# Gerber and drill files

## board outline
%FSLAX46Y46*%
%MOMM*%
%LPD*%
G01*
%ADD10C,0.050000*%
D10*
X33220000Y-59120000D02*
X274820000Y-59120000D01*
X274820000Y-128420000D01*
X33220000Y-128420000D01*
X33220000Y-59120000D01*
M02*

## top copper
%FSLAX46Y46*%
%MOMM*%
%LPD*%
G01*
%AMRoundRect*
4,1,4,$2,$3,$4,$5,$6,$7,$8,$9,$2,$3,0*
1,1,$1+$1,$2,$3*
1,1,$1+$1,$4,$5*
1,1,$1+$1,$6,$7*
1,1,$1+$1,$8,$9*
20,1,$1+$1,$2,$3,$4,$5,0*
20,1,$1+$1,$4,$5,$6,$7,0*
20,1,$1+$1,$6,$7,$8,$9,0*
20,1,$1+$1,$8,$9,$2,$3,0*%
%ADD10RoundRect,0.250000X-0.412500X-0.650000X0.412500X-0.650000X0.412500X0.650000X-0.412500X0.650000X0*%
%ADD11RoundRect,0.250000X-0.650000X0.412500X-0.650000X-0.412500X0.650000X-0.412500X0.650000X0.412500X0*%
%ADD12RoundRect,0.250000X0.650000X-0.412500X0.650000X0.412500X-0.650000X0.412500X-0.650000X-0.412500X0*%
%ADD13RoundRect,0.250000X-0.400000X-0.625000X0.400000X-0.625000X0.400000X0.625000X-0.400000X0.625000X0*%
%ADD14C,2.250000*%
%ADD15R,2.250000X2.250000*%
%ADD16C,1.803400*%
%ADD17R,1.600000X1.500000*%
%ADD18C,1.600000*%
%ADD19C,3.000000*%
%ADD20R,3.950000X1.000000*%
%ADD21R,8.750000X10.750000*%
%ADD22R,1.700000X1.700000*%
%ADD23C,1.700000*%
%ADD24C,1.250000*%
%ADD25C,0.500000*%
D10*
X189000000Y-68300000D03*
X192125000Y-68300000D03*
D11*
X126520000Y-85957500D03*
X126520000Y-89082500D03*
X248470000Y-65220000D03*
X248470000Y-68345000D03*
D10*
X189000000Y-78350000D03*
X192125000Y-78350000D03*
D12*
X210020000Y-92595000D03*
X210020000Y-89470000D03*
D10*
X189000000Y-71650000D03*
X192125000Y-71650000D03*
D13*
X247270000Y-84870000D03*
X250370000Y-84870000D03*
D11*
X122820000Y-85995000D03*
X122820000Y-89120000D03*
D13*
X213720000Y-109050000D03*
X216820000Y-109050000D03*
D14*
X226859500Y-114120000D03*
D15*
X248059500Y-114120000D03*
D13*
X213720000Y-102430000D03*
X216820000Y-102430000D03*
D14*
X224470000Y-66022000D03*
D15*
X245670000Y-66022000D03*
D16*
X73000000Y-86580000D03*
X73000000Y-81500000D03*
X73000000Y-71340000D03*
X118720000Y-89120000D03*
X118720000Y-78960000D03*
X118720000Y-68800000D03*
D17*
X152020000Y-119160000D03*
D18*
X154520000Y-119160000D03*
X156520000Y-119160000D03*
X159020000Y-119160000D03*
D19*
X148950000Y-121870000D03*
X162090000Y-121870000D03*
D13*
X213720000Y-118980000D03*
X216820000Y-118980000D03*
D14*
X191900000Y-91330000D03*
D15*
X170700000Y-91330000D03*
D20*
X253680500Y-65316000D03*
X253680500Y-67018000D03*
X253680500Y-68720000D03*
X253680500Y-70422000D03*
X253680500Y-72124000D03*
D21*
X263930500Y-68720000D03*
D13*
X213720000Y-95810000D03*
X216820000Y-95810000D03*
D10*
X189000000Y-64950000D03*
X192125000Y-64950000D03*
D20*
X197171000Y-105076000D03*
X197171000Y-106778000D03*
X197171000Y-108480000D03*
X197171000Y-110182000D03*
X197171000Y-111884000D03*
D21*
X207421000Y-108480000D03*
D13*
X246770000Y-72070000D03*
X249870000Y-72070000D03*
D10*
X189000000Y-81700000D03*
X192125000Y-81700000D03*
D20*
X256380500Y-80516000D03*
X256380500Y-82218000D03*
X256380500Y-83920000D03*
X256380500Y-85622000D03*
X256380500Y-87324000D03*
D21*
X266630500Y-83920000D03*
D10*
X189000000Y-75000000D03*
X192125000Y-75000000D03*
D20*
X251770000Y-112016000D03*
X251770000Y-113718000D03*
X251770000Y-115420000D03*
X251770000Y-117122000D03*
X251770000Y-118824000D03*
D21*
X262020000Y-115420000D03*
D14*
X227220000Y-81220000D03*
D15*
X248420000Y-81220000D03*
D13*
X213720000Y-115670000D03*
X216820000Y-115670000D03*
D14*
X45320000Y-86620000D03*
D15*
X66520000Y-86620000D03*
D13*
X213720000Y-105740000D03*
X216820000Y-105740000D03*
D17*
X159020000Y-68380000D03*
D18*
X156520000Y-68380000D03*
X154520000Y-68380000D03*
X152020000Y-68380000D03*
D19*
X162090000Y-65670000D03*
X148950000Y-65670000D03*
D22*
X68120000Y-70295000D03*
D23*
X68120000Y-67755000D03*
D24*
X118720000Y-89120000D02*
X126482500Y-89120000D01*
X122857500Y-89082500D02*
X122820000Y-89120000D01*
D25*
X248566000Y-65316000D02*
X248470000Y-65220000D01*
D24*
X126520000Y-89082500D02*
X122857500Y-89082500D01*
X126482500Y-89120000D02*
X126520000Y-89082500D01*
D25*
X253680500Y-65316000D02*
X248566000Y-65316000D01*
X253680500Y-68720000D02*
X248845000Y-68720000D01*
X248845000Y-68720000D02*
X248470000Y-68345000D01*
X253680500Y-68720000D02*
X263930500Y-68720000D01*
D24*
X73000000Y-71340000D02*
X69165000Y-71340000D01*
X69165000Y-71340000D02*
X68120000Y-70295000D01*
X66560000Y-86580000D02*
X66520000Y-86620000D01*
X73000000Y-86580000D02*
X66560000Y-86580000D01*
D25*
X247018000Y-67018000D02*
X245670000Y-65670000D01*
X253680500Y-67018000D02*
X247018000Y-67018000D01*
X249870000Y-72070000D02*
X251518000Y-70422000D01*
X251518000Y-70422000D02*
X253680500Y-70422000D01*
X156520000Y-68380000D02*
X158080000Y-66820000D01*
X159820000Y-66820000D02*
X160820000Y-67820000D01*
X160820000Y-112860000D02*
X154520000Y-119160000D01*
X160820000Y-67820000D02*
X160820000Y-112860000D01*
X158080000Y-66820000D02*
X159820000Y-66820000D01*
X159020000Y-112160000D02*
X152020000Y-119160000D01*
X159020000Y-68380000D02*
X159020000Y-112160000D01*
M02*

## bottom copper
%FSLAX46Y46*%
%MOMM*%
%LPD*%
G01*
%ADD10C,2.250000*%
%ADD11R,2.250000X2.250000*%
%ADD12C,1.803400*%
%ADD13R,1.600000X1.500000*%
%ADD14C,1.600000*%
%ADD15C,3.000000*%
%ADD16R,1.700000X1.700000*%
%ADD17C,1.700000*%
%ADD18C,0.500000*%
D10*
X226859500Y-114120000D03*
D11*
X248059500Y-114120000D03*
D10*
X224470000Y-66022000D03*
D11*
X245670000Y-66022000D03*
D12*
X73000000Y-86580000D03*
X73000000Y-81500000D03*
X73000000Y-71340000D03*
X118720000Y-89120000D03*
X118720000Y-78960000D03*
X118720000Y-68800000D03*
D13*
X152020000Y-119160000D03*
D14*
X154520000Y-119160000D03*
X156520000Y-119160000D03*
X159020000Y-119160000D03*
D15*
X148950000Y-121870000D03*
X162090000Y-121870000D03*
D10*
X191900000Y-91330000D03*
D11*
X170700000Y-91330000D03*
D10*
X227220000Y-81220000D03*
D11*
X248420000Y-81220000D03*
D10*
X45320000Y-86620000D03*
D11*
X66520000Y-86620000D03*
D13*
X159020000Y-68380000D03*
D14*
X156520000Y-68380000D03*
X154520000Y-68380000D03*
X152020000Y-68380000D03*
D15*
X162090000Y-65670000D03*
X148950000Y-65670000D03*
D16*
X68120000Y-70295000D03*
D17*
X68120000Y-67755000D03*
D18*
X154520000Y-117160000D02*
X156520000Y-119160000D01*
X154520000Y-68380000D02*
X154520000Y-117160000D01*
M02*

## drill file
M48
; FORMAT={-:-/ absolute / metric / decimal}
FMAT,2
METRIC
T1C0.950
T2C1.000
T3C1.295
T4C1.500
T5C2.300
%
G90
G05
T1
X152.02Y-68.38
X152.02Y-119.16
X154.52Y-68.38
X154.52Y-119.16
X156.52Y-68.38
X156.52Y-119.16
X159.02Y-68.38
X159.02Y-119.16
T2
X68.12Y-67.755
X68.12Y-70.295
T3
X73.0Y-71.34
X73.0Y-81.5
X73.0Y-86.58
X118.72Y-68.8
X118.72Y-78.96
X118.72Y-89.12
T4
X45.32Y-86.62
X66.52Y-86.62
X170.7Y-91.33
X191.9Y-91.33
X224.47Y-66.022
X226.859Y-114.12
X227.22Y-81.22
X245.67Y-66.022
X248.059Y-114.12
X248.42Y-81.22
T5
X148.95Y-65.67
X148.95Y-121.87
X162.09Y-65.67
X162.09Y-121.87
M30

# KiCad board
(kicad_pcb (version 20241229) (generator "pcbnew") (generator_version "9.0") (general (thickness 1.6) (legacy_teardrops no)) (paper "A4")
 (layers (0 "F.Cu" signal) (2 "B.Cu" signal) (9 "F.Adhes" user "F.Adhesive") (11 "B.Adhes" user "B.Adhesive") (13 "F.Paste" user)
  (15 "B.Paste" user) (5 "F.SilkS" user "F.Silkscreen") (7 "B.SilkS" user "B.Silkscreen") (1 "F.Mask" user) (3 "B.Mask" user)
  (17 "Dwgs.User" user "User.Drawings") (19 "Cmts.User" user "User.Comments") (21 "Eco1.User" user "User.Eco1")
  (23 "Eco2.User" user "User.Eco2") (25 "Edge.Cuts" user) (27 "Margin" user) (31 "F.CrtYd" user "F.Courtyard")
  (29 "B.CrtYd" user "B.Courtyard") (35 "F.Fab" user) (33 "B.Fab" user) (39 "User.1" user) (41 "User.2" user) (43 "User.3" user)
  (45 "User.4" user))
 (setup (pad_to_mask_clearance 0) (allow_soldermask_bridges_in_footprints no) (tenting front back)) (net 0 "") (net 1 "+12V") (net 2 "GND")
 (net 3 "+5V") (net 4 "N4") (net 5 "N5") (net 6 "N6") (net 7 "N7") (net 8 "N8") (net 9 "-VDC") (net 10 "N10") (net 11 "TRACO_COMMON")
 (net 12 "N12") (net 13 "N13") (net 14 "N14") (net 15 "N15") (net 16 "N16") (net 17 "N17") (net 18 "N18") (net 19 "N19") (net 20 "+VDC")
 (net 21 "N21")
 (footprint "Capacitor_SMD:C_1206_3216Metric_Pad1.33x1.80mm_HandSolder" (layer "F.Cu") (at 190.5625 68.3)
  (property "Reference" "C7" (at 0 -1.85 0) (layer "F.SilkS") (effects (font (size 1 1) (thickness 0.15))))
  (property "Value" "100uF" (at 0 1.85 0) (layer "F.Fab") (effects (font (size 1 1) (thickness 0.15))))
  (pad "1" smd roundrect (at -1.5625 0) (size 1.325 1.8) (layers "F.Cu" "F.Mask" "F.Paste") (roundrect_rratio 0.188679) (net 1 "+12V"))
  (pad "2" smd roundrect (at 1.5625 0) (size 1.325 1.8) (layers "F.Cu" "F.Mask" "F.Paste") (roundrect_rratio 0.188679) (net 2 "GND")))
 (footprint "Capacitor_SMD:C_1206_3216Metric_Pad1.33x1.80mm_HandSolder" (layer "F.Cu") (at 126.52 87.52 -90)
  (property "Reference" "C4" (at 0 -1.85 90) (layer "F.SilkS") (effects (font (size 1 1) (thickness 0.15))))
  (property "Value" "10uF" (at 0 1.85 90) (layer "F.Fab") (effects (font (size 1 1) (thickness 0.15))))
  (pad "1" smd roundrect (at -1.5625 0 270) (size 1.325 1.8) (layers "F.Cu" "F.Mask" "F.Paste") (roundrect_rratio 0.188679) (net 2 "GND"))
  (pad "2" smd roundrect (at 1.5625 0 270) (size 1.325 1.8) (layers "F.Cu" "F.Mask" "F.Paste") (roundrect_rratio 0.188679) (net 1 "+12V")))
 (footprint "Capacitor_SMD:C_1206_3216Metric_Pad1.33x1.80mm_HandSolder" (layer "F.Cu") (at 248.47 66.7825 -90)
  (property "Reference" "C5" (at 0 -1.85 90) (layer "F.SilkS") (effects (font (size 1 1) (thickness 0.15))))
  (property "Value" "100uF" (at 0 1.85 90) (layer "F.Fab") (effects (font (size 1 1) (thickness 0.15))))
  (pad "1" smd roundrect (at -1.5625 0 270) (size 1.325 1.8) (layers "F.Cu" "F.Mask" "F.Paste") (roundrect_rratio 0.188679) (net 1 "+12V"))
  (pad "2" smd roundrect (at 1.5625 0 270) (size 1.325 1.8) (layers "F.Cu" "F.Mask" "F.Paste") (roundrect_rratio 0.188679) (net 2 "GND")))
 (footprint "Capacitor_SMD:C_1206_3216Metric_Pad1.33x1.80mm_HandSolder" (layer "F.Cu") (at 190.5625 78.35)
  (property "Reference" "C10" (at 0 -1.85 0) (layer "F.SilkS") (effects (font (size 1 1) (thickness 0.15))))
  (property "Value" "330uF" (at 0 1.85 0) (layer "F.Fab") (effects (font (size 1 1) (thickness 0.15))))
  (pad "1" smd roundrect (at -1.5625 0) (size 1.325 1.8) (layers "F.Cu" "F.Mask" "F.Paste") (roundrect_rratio 0.188679) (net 2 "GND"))
  (pad "2" smd roundrect (at 1.5625 0) (size 1.325 1.8) (layers "F.Cu" "F.Mask" "F.Paste") (roundrect_rratio 0.188679) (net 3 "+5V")))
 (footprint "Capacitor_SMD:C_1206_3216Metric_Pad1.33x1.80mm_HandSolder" (layer "F.Cu") (at 210.02 91.0325 90)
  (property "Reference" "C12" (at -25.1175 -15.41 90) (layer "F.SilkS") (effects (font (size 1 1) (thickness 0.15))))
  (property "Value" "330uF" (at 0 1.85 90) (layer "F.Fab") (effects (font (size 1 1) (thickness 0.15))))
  (pad "1" smd roundrect (at -1.5625 0 90) (size 1.325 1.8) (layers "F.Cu" "F.Mask" "F.Paste") (roundrect_rratio 0.188679) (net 2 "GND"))
  (pad "2" smd roundrect (at 1.5625 0 90) (size 1.325 1.8) (layers "F.Cu" "F.Mask" "F.Paste") (roundrect_rratio 0.188679) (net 3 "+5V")))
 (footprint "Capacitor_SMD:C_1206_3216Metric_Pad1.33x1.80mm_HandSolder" (layer "F.Cu") (at 190.5625 71.65)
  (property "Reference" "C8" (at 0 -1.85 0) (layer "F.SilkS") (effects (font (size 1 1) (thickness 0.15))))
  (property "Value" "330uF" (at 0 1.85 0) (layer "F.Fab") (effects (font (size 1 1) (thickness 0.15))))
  (pad "1" smd roundrect (at -1.5625 0) (size 1.325 1.8) (layers "F.Cu" "F.Mask" "F.Paste") (roundrect_rratio 0.188679) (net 2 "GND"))
  (pad "2" smd roundrect (at 1.5625 0) (size 1.325 1.8) (layers "F.Cu" "F.Mask" "F.Paste") (roundrect_rratio 0.188679) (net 3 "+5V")))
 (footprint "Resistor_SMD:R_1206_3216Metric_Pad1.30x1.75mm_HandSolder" (layer "F.Cu") (at 248.82 84.87)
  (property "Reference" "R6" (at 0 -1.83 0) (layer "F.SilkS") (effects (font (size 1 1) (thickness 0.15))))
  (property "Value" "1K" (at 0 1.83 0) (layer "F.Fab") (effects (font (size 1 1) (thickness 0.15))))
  (pad "1" smd roundrect (at -1.55 0) (size 1.3 1.75) (layers "F.Cu" "F.Mask" "F.Paste") (roundrect_rratio 0.192308) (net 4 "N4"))
  (pad "2" smd roundrect (at 1.55 0) (size 1.3 1.75) (layers "F.Cu" "F.Mask" "F.Paste") (roundrect_rratio 0.192308) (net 2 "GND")))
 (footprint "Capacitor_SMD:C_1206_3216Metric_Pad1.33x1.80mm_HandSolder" (layer "F.Cu") (at 122.82 87.5575 -90)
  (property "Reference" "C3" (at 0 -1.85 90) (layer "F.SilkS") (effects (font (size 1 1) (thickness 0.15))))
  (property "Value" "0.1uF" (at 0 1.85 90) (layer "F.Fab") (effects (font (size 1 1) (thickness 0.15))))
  (pad "1" smd roundrect (at -1.5625 0 270) (size 1.325 1.8) (layers "F.Cu" "F.Mask" "F.Paste") (roundrect_rratio 0.188679) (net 2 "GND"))
  (pad "2" smd roundrect (at 1.5625 0 270) (size 1.325 1.8) (layers "F.Cu" "F.Mask" "F.Paste") (roundrect_rratio 0.188679) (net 1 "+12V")))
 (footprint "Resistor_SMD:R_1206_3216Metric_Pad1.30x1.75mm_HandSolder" (layer "F.Cu") (at 215.27 109.05)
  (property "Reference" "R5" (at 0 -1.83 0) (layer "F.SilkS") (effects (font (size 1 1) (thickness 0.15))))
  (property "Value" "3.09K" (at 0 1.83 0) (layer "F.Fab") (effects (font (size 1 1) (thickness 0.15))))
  (pad "1" smd roundrect (at -1.55 0) (size 1.3 1.75) (layers "F.Cu" "F.Mask" "F.Paste") (roundrect_rratio 0.192308) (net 3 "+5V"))
  (pad "2" smd roundrect (at 1.55 0) (size 1.3 1.75) (layers "F.Cu" "F.Mask" "F.Paste") (roundrect_rratio 0.192308) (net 4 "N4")))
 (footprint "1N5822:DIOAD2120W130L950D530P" (layer "F.Cu") (at 237.4595 114.12 180)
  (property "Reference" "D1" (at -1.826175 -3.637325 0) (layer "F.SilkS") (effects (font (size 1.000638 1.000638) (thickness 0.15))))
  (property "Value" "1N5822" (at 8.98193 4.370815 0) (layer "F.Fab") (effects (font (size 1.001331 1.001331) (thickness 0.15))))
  (pad "A" thru_hole circle (at 10.6 0 180) (size 2.25 2.25) (drill 1.5) (layers "*.Cu" "*.Mask") (remove_unused_layers no) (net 2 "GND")
   (solder_mask_margin 0.102))
  (pad "C" thru_hole rect (at -10.6 0 180) (size 2.25 2.25) (drill 1.5) (layers "*.Cu" "*.Mask") (remove_unused_layers no) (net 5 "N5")
   (solder_mask_margin 0.102)))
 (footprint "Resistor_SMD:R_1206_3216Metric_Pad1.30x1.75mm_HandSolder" (layer "F.Cu") (at 215.27 102.43)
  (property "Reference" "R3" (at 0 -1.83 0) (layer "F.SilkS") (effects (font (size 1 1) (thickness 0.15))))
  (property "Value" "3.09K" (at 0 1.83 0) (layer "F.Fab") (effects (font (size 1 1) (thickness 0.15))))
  (pad "1" smd roundrect (at -1.55 0) (size 1.3 1.75) (layers "F.Cu" "F.Mask" "F.Paste") (roundrect_rratio 0.192308) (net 3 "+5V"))
  (pad "2" smd roundrect (at 1.55 0) (size 1.3 1.75) (layers "F.Cu" "F.Mask" "F.Paste") (roundrect_rratio 0.192308) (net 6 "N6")))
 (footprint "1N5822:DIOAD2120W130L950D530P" (layer "F.Cu") (at 235.07 66.022 180)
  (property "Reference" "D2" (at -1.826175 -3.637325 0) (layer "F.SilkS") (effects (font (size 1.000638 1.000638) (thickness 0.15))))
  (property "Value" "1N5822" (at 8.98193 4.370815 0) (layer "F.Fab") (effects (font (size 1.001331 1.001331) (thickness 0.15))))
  (pad "A" thru_hole circle (at 10.6 0 180) (size 2.25 2.25) (drill 1.5) (layers "*.Cu" "*.Mask") (remove_unused_layers no) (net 2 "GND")
   (solder_mask_margin 0.102))
  (pad "C" thru_hole rect (at -10.6 0 180) (size 2.25 2.25) (drill 1.5) (layers "*.Cu" "*.Mask") (remove_unused_layers no) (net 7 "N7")
   (solder_mask_margin 0.102)))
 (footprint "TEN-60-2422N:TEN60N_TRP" (layer "F.Cu") (at 73 86.58)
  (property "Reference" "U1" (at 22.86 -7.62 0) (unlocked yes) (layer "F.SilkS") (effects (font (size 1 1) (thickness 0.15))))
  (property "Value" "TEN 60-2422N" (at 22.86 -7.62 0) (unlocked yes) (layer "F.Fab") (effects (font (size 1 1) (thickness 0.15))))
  (pad "1" thru_hole circle (at 0 0) (size 1.8034 1.8034) (drill 1.2954) (layers "*.Cu" "*.Mask") (remove_unused_layers no) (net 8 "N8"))
  (pad "2" thru_hole circle (at 0 -5.08) (size 1.8034 1.8034) (drill 1.2954) (layers "*.Cu" "*.Mask") (remove_unused_layers no)
   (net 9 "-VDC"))
  (pad "3" thru_hole circle (at 0 -15.24) (size 1.8034 1.8034) (drill 1.2954) (layers "*.Cu" "*.Mask") (remove_unused_layers no)
   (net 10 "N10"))
  (pad "4" thru_hole circle (at 45.72 2.54) (size 1.8034 1.8034) (drill 1.2954) (layers "*.Cu" "*.Mask") (remove_unused_layers no)
   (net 1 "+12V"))
  (pad "5" thru_hole circle (at 45.72 -7.62) (size 1.8034 1.8034) (drill 1.2954) (layers "*.Cu" "*.Mask") (remove_unused_layers no)
   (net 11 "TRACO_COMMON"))
  (pad "6" thru_hole circle (at 45.72 -17.78) (size 1.8034 1.8034) (drill 1.2954) (layers "*.Cu" "*.Mask") (remove_unused_layers no)
   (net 2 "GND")))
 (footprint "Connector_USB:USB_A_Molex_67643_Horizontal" (layer "F.Cu") (at 152.02 119.16)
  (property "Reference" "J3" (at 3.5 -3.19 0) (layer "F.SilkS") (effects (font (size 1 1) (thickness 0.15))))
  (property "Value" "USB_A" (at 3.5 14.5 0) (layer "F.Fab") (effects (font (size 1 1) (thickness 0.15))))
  (pad "1" thru_hole rect (at 0 0) (size 1.6 1.5) (drill 0.95) (layers "*.Cu" "*.Mask") (remove_unused_layers no) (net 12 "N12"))
  (pad "2" thru_hole circle (at 2.5 0) (size 1.6 1.6) (drill 0.95) (layers "*.Cu" "*.Mask") (remove_unused_layers no) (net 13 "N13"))
  (pad "3" thru_hole circle (at 4.5 0) (size 1.6 1.6) (drill 0.95) (layers "*.Cu" "*.Mask") (remove_unused_layers no) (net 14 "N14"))
  (pad "4" thru_hole circle (at 7 0) (size 1.6 1.6) (drill 0.95) (layers "*.Cu" "*.Mask") (remove_unused_layers no) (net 2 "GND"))
  (pad "5" thru_hole circle (at -3.07 2.71) (size 3 3) (drill 2.3) (layers "*.Cu" "*.Mask") (remove_unused_layers no) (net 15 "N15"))
  (pad "5" thru_hole circle (at 10.07 2.71) (size 3 3) (drill 2.3) (layers "*.Cu" "*.Mask") (remove_unused_layers no) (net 15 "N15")))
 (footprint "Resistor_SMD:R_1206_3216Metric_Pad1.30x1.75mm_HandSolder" (layer "F.Cu") (at 215.27 118.98)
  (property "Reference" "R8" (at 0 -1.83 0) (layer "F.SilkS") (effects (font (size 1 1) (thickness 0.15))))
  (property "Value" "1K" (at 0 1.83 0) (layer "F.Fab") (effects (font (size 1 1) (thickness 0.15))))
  (pad "1" smd roundrect (at -1.55 0) (size 1.3 1.75) (layers "F.Cu" "F.Mask" "F.Paste") (roundrect_rratio 0.192308) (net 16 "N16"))
  (pad "2" smd roundrect (at 1.55 0) (size 1.3 1.75) (layers "F.Cu" "F.Mask" "F.Paste") (roundrect_rratio 0.192308) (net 2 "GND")))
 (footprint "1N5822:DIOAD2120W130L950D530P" (layer "F.Cu") (at 181.3 91.33)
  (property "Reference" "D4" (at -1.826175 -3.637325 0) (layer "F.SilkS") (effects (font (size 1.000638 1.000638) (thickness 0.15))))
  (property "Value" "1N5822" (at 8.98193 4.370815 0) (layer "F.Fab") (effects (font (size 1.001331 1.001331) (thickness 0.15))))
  (pad "A" thru_hole circle (at 10.6 0) (size 2.25 2.25) (drill 1.5) (layers "*.Cu" "*.Mask") (remove_unused_layers no) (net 2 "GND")
   (solder_mask_margin 0.102))
  (pad "C" thru_hole rect (at -10.6 0) (size 2.25 2.25) (drill 1.5) (layers "*.Cu" "*.Mask") (remove_unused_layers no) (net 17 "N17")
   (solder_mask_margin 0.102)))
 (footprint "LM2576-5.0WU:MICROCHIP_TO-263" (layer "F.Cu") (at 266.2095 68.72)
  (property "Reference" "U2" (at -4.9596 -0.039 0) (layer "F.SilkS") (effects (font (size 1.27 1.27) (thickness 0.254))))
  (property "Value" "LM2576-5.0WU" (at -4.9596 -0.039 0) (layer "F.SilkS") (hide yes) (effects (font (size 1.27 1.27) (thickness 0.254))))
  (pad "1" smd rect (at -12.529 -3.404 90) (size 1 3.95) (layers "F.Cu" "F.Mask" "F.Paste") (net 1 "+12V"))
  (pad "2" smd rect (at -12.529 -1.702 90) (size 1 3.95) (layers "F.Cu" "F.Mask" "F.Paste") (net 7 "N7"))
  (pad "3" smd rect (at -12.529 0 90) (size 1 3.95) (layers "F.Cu" "F.Mask" "F.Paste") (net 2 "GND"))
  (pad "4" smd rect (at -12.529 1.702 90) (size 1 3.95) (layers "F.Cu" "F.Mask" "F.Paste") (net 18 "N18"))
  (pad "5" smd rect (at -12.529 3.404 90) (size 1 3.95) (layers "F.Cu" "F.Mask" "F.Paste") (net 2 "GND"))
  (pad "6" smd rect (at -2.279 0) (size 8.75 10.75) (layers "F.Cu" "F.Mask" "F.Paste") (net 2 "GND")))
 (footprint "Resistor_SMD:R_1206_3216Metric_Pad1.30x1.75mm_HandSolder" (layer "F.Cu") (at 215.27 95.81)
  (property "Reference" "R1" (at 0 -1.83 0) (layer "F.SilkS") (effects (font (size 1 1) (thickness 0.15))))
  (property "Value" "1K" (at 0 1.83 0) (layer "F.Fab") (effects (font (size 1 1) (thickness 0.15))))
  (pad "1" smd roundrect (at -1.55 0) (size 1.3 1.75) (layers "F.Cu" "F.Mask" "F.Paste") (roundrect_rratio 0.192308) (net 18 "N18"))
  (pad "2" smd roundrect (at 1.55 0) (size 1.3 1.75) (layers "F.Cu" "F.Mask" "F.Paste") (roundrect_rratio 0.192308) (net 2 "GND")))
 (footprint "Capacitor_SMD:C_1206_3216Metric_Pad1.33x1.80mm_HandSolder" (layer "F.Cu") (at 190.5625 64.95)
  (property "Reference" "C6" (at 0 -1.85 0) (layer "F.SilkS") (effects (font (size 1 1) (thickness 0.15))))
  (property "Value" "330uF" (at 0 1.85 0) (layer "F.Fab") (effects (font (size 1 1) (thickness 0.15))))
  (pad "1" smd roundrect (at -1.5625 0) (size 1.325 1.8) (layers "F.Cu" "F.Mask" "F.Paste") (roundrect_rratio 0.188679) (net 2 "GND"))
  (pad "2" smd roundrect (at 1.5625 0) (size 1.325 1.8) (layers "F.Cu" "F.Mask" "F.Paste") (roundrect_rratio 0.188679) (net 3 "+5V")))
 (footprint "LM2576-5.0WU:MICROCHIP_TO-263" (layer "F.Cu") (at 209.7 108.48)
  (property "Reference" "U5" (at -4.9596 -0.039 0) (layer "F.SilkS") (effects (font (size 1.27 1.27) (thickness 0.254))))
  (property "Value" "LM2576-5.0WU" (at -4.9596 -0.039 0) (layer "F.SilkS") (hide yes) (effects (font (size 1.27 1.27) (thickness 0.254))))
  (pad "1" smd rect (at -12.529 -3.404 90) (size 1 3.95) (layers "F.Cu" "F.Mask" "F.Paste") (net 1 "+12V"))
  (pad "2" smd rect (at -12.529 -1.702 90) (size 1 3.95) (layers "F.Cu" "F.Mask" "F.Paste") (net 17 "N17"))
  (pad "3" smd rect (at -12.529 0 90) (size 1 3.95) (layers "F.Cu" "F.Mask" "F.Paste") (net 2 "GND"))
  (pad "4" smd rect (at -12.529 1.702 90) (size 1 3.95) (layers "F.Cu" "F.Mask" "F.Paste") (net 16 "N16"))
  (pad "5" smd rect (at -12.529 3.404 90) (size 1 3.95) (layers "F.Cu" "F.Mask" "F.Paste") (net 2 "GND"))
  (pad "6" smd rect (at -2.279 0) (size 8.75 10.75) (layers "F.Cu" "F.Mask" "F.Paste") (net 2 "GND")))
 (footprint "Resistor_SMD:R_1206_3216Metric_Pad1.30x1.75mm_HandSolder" (layer "F.Cu") (at 248.32 72.07)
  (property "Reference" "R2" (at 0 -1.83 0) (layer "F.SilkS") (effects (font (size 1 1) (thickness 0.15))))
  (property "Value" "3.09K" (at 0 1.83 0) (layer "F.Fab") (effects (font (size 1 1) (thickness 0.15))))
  (pad "1" smd roundrect (at -1.55 0) (size 1.3 1.75) (layers "F.Cu" "F.Mask" "F.Paste") (roundrect_rratio 0.192308) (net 3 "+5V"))
  (pad "2" smd roundrect (at 1.55 0) (size 1.3 1.75) (layers "F.Cu" "F.Mask" "F.Paste") (roundrect_rratio 0.192308) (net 18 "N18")))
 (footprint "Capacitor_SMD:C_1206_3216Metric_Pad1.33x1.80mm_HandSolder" (layer "F.Cu") (at 190.5625 81.7)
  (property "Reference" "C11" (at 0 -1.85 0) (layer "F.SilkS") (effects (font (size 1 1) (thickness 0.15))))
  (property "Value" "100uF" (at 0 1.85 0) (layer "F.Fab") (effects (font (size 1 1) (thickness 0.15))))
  (pad "1" smd roundrect (at -1.5625 0) (size 1.325 1.8) (layers "F.Cu" "F.Mask" "F.Paste") (roundrect_rratio 0.188679) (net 1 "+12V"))
  (pad "2" smd roundrect (at 1.5625 0) (size 1.325 1.8) (layers "F.Cu" "F.Mask" "F.Paste") (roundrect_rratio 0.188679) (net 2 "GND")))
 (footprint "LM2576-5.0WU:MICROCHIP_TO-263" (layer "F.Cu") (at 268.9095 83.92)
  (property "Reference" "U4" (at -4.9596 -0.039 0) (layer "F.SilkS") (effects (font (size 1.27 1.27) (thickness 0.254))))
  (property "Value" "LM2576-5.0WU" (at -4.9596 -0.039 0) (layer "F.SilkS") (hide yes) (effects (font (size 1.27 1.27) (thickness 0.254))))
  (pad "1" smd rect (at -12.529 -3.404 90) (size 1 3.95) (layers "F.Cu" "F.Mask" "F.Paste") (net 1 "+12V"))
  (pad "2" smd rect (at -12.529 -1.702 90) (size 1 3.95) (layers "F.Cu" "F.Mask" "F.Paste") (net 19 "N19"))
  (pad "3" smd rect (at -12.529 0 90) (size 1 3.95) (layers "F.Cu" "F.Mask" "F.Paste") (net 2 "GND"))
  (pad "4" smd rect (at -12.529 1.702 90) (size 1 3.95) (layers "F.Cu" "F.Mask" "F.Paste") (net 4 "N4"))
  (pad "5" smd rect (at -12.529 3.404 90) (size 1 3.95) (layers "F.Cu" "F.Mask" "F.Paste") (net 2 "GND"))
  (pad "6" smd rect (at -2.279 0) (size 8.75 10.75) (layers "F.Cu" "F.Mask" "F.Paste") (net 2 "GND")))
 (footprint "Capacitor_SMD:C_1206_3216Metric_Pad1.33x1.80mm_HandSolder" (layer "F.Cu") (at 190.5625 75)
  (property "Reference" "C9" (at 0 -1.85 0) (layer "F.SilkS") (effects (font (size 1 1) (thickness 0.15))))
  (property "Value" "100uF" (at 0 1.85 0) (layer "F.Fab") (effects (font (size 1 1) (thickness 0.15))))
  (pad "1" smd roundrect (at -1.5625 0) (size 1.325 1.8) (layers "F.Cu" "F.Mask" "F.Paste") (roundrect_rratio 0.188679) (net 1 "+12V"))
  (pad "2" smd roundrect (at 1.5625 0) (size 1.325 1.8) (layers "F.Cu" "F.Mask" "F.Paste") (roundrect_rratio 0.188679) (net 2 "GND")))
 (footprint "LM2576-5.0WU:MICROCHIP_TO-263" (layer "F.Cu") (at 264.299 115.42)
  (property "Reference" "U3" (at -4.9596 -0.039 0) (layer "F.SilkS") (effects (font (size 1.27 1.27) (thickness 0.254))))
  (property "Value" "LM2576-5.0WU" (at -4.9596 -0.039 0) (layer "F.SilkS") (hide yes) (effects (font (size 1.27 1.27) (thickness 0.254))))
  (pad "1" smd rect (at -12.529 -3.404 90) (size 1 3.95) (layers "F.Cu" "F.Mask" "F.Paste") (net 1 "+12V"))
  (pad "2" smd rect (at -12.529 -1.702 90) (size 1 3.95) (layers "F.Cu" "F.Mask" "F.Paste") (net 5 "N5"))
  (pad "3" smd rect (at -12.529 0 90) (size 1 3.95) (layers "F.Cu" "F.Mask" "F.Paste") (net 2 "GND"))
  (pad "4" smd rect (at -12.529 1.702 90) (size 1 3.95) (layers "F.Cu" "F.Mask" "F.Paste") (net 6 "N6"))
  (pad "5" smd rect (at -12.529 3.404 90) (size 1 3.95) (layers "F.Cu" "F.Mask" "F.Paste") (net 2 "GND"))
  (pad "6" smd rect (at -2.279 0) (size 8.75 10.75) (layers "F.Cu" "F.Mask" "F.Paste") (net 2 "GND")))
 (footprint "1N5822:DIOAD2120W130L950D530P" (layer "F.Cu") (at 237.82 81.22 180)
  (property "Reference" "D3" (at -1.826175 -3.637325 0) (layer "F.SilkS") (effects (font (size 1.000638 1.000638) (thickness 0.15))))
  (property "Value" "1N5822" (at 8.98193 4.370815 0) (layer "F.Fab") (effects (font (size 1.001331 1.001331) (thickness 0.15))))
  (pad "A" thru_hole circle (at 10.6 0 180) (size 2.25 2.25) (drill 1.5) (layers "*.Cu" "*.Mask") (remove_unused_layers no) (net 2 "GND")
   (solder_mask_margin 0.102))
  (pad "C" thru_hole rect (at -10.6 0 180) (size 2.25 2.25) (drill 1.5) (layers "*.Cu" "*.Mask") (remove_unused_layers no) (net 19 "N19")
   (solder_mask_margin 0.102)))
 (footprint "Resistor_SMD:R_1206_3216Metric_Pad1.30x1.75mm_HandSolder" (layer "F.Cu") (at 215.27 115.67)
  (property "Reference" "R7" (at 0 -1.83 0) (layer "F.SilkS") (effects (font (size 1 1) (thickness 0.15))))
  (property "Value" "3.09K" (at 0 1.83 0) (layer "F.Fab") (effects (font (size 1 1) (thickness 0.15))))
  (pad "1" smd roundrect (at -1.55 0) (size 1.3 1.75) (layers "F.Cu" "F.Mask" "F.Paste") (roundrect_rratio 0.192308) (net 3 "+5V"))
  (pad "2" smd roundrect (at 1.55 0) (size 1.3 1.75) (layers "F.Cu" "F.Mask" "F.Paste") (roundrect_rratio 0.192308) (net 16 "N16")))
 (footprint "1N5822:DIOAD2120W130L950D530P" (layer "F.Cu") (at 55.92 86.62 180)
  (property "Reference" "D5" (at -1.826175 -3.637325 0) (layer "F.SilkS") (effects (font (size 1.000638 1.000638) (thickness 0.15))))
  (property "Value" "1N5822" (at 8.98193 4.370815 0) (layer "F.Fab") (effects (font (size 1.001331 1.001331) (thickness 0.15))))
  (pad "A" thru_hole circle (at 10.6 0 180) (size 2.25 2.25) (drill 1.5) (layers "*.Cu" "*.Mask") (remove_unused_layers no) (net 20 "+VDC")
   (solder_mask_margin 0.102))
  (pad "C" thru_hole rect (at -10.6 0 180) (size 2.25 2.25) (drill 1.5) (layers "*.Cu" "*.Mask") (remove_unused_layers no) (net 8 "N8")
   (solder_mask_margin 0.102)))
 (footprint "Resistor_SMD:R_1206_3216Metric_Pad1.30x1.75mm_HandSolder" (layer "F.Cu") (at 215.27 105.74)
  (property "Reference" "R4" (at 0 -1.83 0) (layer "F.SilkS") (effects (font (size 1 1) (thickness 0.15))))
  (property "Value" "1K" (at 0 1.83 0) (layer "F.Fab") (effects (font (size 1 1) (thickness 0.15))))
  (pad "1" smd roundrect (at -1.55 0) (size 1.3 1.75) (layers "F.Cu" "F.Mask" "F.Paste") (roundrect_rratio 0.192308) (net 6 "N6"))
  (pad "2" smd roundrect (at 1.55 0) (size 1.3 1.75) (layers "F.Cu" "F.Mask" "F.Paste") (roundrect_rratio 0.192308) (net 2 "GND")))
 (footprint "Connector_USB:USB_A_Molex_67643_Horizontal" (layer "F.Cu") (at 159.02 68.38 180)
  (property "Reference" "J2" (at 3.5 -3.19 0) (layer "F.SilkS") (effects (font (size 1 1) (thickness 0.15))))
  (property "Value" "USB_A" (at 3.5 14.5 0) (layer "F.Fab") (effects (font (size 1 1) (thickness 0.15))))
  (pad "1" thru_hole rect (at 0 0 180) (size 1.6 1.5) (drill 0.95) (layers "*.Cu" "*.Mask") (remove_unused_layers no) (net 12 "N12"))
  (pad "2" thru_hole circle (at 2.5 0 180) (size 1.6 1.6) (drill 0.95) (layers "*.Cu" "*.Mask") (remove_unused_layers no) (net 13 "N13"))
  (pad "3" thru_hole circle (at 4.5 0 180) (size 1.6 1.6) (drill 0.95) (layers "*.Cu" "*.Mask") (remove_unused_layers no) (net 14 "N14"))
  (pad "4" thru_hole circle (at 7 0 180) (size 1.6 1.6) (drill 0.95) (layers "*.Cu" "*.Mask") (remove_unused_layers no) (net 2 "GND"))
  (pad "5" thru_hole circle (at -3.07 2.71 180) (size 3 3) (drill 2.3) (layers "*.Cu" "*.Mask") (remove_unused_layers no) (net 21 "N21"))
  (pad "5" thru_hole circle (at 10.07 2.71 180) (size 3 3) (drill 2.3) (layers "*.Cu" "*.Mask") (remove_unused_layers no) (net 21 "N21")))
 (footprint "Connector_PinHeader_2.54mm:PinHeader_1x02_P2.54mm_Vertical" (layer "B.Cu") (at 68.12 70.295)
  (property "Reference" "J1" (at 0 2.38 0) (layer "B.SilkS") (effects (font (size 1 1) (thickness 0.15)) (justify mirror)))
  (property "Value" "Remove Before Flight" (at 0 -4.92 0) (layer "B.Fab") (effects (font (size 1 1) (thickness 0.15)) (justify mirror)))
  (pad "1" thru_hole rect (at 0 0) (size 1.7 1.7) (drill 1) (layers "*.Cu" "*.Mask") (remove_unused_layers no) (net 10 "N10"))
  (pad "2" thru_hole circle (at 0 -2.54) (size 1.7 1.7) (drill 1) (layers "*.Cu" "*.Mask") (remove_unused_layers no) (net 9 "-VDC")))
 (gr_rect (start 33.22 59.12) (end 274.82 128.42) (stroke (width 0.05) (type default)) (fill no) (layer "Edge.Cuts"))
 (segment (start 118.72 89.12) (end 126.4825 89.12) (width 1.25) (layer "F.Cu") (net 1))
 (segment (start 122.8575 89.0825) (end 122.82 89.12) (width 1.25) (layer "F.Cu") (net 1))
 (segment (start 248.566 65.316) (end 248.47 65.22) (width 0.5) (layer "F.Cu") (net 1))
 (segment (start 126.52 89.0825) (end 122.8575 89.0825) (width 1.25) (layer "F.Cu") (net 1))
 (segment (start 126.4825 89.12) (end 126.52 89.0825) (width 1.25) (layer "F.Cu") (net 1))
 (segment (start 253.6805 65.316) (end 248.566 65.316) (width 0.5) (layer "F.Cu") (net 1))
 (segment (start 253.6805 68.72) (end 248.845 68.72) (width 0.5) (layer "F.Cu") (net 2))
 (segment (start 248.845 68.72) (end 248.47 68.345) (width 0.5) (layer "F.Cu") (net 2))
 (segment (start 253.6805 68.72) (end 263.9305 68.72) (width 0.5) (layer "F.Cu") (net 2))
 (segment (start 73 71.34) (end 69.165 71.34) (width 1.25) (layer "F.Cu") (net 10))
 (segment (start 69.165 71.34) (end 68.12 70.295) (width 1.25) (layer "F.Cu") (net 10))
 (segment (start 66.56 86.58) (end 66.52 86.62) (width 1.25) (layer "F.Cu") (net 8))
 (segment (start 73 86.58) (end 66.56 86.58) (width 1.25) (layer "F.Cu") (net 8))
 (segment (start 247.018 67.018) (end 245.67 65.67) (width 0.5) (layer "F.Cu") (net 7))
 (segment (start 253.6805 67.018) (end 247.018 67.018) (width 0.5) (layer "F.Cu") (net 7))
 (segment (start 249.87 72.07) (end 251.518 70.422) (width 0.5) (layer "F.Cu") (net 18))
 (segment (start 251.518 70.422) (end 253.6805 70.422) (width 0.5) (layer "F.Cu") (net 18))
 (segment (start 156.52 68.38) (end 158.08 66.82) (width 0.5) (layer "F.Cu") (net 13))
 (segment (start 159.82 66.82) (end 160.82 67.82) (width 0.5) (layer "F.Cu") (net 13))
 (segment (start 160.82 112.86) (end 154.52 119.16) (width 0.5) (layer "F.Cu") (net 13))
 (segment (start 160.82 67.82) (end 160.82 112.86) (width 0.5) (layer "F.Cu") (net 13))
 (segment (start 158.08 66.82) (end 159.82 66.82) (width 0.5) (layer "F.Cu") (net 13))
 (segment (start 154.52 117.16) (end 156.52 119.16) (width 0.5) (layer "B.Cu") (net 14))
 (segment (start 154.52 68.38) (end 154.52 117.16) (width 0.5) (layer "B.Cu") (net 14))
 (segment (start 159.02 112.16) (end 152.02 119.16) (width 0.5) (layer "F.Cu") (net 12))
 (segment (start 159.02 68.38) (end 159.02 112.16) (width 0.5) (layer "F.Cu") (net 12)))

